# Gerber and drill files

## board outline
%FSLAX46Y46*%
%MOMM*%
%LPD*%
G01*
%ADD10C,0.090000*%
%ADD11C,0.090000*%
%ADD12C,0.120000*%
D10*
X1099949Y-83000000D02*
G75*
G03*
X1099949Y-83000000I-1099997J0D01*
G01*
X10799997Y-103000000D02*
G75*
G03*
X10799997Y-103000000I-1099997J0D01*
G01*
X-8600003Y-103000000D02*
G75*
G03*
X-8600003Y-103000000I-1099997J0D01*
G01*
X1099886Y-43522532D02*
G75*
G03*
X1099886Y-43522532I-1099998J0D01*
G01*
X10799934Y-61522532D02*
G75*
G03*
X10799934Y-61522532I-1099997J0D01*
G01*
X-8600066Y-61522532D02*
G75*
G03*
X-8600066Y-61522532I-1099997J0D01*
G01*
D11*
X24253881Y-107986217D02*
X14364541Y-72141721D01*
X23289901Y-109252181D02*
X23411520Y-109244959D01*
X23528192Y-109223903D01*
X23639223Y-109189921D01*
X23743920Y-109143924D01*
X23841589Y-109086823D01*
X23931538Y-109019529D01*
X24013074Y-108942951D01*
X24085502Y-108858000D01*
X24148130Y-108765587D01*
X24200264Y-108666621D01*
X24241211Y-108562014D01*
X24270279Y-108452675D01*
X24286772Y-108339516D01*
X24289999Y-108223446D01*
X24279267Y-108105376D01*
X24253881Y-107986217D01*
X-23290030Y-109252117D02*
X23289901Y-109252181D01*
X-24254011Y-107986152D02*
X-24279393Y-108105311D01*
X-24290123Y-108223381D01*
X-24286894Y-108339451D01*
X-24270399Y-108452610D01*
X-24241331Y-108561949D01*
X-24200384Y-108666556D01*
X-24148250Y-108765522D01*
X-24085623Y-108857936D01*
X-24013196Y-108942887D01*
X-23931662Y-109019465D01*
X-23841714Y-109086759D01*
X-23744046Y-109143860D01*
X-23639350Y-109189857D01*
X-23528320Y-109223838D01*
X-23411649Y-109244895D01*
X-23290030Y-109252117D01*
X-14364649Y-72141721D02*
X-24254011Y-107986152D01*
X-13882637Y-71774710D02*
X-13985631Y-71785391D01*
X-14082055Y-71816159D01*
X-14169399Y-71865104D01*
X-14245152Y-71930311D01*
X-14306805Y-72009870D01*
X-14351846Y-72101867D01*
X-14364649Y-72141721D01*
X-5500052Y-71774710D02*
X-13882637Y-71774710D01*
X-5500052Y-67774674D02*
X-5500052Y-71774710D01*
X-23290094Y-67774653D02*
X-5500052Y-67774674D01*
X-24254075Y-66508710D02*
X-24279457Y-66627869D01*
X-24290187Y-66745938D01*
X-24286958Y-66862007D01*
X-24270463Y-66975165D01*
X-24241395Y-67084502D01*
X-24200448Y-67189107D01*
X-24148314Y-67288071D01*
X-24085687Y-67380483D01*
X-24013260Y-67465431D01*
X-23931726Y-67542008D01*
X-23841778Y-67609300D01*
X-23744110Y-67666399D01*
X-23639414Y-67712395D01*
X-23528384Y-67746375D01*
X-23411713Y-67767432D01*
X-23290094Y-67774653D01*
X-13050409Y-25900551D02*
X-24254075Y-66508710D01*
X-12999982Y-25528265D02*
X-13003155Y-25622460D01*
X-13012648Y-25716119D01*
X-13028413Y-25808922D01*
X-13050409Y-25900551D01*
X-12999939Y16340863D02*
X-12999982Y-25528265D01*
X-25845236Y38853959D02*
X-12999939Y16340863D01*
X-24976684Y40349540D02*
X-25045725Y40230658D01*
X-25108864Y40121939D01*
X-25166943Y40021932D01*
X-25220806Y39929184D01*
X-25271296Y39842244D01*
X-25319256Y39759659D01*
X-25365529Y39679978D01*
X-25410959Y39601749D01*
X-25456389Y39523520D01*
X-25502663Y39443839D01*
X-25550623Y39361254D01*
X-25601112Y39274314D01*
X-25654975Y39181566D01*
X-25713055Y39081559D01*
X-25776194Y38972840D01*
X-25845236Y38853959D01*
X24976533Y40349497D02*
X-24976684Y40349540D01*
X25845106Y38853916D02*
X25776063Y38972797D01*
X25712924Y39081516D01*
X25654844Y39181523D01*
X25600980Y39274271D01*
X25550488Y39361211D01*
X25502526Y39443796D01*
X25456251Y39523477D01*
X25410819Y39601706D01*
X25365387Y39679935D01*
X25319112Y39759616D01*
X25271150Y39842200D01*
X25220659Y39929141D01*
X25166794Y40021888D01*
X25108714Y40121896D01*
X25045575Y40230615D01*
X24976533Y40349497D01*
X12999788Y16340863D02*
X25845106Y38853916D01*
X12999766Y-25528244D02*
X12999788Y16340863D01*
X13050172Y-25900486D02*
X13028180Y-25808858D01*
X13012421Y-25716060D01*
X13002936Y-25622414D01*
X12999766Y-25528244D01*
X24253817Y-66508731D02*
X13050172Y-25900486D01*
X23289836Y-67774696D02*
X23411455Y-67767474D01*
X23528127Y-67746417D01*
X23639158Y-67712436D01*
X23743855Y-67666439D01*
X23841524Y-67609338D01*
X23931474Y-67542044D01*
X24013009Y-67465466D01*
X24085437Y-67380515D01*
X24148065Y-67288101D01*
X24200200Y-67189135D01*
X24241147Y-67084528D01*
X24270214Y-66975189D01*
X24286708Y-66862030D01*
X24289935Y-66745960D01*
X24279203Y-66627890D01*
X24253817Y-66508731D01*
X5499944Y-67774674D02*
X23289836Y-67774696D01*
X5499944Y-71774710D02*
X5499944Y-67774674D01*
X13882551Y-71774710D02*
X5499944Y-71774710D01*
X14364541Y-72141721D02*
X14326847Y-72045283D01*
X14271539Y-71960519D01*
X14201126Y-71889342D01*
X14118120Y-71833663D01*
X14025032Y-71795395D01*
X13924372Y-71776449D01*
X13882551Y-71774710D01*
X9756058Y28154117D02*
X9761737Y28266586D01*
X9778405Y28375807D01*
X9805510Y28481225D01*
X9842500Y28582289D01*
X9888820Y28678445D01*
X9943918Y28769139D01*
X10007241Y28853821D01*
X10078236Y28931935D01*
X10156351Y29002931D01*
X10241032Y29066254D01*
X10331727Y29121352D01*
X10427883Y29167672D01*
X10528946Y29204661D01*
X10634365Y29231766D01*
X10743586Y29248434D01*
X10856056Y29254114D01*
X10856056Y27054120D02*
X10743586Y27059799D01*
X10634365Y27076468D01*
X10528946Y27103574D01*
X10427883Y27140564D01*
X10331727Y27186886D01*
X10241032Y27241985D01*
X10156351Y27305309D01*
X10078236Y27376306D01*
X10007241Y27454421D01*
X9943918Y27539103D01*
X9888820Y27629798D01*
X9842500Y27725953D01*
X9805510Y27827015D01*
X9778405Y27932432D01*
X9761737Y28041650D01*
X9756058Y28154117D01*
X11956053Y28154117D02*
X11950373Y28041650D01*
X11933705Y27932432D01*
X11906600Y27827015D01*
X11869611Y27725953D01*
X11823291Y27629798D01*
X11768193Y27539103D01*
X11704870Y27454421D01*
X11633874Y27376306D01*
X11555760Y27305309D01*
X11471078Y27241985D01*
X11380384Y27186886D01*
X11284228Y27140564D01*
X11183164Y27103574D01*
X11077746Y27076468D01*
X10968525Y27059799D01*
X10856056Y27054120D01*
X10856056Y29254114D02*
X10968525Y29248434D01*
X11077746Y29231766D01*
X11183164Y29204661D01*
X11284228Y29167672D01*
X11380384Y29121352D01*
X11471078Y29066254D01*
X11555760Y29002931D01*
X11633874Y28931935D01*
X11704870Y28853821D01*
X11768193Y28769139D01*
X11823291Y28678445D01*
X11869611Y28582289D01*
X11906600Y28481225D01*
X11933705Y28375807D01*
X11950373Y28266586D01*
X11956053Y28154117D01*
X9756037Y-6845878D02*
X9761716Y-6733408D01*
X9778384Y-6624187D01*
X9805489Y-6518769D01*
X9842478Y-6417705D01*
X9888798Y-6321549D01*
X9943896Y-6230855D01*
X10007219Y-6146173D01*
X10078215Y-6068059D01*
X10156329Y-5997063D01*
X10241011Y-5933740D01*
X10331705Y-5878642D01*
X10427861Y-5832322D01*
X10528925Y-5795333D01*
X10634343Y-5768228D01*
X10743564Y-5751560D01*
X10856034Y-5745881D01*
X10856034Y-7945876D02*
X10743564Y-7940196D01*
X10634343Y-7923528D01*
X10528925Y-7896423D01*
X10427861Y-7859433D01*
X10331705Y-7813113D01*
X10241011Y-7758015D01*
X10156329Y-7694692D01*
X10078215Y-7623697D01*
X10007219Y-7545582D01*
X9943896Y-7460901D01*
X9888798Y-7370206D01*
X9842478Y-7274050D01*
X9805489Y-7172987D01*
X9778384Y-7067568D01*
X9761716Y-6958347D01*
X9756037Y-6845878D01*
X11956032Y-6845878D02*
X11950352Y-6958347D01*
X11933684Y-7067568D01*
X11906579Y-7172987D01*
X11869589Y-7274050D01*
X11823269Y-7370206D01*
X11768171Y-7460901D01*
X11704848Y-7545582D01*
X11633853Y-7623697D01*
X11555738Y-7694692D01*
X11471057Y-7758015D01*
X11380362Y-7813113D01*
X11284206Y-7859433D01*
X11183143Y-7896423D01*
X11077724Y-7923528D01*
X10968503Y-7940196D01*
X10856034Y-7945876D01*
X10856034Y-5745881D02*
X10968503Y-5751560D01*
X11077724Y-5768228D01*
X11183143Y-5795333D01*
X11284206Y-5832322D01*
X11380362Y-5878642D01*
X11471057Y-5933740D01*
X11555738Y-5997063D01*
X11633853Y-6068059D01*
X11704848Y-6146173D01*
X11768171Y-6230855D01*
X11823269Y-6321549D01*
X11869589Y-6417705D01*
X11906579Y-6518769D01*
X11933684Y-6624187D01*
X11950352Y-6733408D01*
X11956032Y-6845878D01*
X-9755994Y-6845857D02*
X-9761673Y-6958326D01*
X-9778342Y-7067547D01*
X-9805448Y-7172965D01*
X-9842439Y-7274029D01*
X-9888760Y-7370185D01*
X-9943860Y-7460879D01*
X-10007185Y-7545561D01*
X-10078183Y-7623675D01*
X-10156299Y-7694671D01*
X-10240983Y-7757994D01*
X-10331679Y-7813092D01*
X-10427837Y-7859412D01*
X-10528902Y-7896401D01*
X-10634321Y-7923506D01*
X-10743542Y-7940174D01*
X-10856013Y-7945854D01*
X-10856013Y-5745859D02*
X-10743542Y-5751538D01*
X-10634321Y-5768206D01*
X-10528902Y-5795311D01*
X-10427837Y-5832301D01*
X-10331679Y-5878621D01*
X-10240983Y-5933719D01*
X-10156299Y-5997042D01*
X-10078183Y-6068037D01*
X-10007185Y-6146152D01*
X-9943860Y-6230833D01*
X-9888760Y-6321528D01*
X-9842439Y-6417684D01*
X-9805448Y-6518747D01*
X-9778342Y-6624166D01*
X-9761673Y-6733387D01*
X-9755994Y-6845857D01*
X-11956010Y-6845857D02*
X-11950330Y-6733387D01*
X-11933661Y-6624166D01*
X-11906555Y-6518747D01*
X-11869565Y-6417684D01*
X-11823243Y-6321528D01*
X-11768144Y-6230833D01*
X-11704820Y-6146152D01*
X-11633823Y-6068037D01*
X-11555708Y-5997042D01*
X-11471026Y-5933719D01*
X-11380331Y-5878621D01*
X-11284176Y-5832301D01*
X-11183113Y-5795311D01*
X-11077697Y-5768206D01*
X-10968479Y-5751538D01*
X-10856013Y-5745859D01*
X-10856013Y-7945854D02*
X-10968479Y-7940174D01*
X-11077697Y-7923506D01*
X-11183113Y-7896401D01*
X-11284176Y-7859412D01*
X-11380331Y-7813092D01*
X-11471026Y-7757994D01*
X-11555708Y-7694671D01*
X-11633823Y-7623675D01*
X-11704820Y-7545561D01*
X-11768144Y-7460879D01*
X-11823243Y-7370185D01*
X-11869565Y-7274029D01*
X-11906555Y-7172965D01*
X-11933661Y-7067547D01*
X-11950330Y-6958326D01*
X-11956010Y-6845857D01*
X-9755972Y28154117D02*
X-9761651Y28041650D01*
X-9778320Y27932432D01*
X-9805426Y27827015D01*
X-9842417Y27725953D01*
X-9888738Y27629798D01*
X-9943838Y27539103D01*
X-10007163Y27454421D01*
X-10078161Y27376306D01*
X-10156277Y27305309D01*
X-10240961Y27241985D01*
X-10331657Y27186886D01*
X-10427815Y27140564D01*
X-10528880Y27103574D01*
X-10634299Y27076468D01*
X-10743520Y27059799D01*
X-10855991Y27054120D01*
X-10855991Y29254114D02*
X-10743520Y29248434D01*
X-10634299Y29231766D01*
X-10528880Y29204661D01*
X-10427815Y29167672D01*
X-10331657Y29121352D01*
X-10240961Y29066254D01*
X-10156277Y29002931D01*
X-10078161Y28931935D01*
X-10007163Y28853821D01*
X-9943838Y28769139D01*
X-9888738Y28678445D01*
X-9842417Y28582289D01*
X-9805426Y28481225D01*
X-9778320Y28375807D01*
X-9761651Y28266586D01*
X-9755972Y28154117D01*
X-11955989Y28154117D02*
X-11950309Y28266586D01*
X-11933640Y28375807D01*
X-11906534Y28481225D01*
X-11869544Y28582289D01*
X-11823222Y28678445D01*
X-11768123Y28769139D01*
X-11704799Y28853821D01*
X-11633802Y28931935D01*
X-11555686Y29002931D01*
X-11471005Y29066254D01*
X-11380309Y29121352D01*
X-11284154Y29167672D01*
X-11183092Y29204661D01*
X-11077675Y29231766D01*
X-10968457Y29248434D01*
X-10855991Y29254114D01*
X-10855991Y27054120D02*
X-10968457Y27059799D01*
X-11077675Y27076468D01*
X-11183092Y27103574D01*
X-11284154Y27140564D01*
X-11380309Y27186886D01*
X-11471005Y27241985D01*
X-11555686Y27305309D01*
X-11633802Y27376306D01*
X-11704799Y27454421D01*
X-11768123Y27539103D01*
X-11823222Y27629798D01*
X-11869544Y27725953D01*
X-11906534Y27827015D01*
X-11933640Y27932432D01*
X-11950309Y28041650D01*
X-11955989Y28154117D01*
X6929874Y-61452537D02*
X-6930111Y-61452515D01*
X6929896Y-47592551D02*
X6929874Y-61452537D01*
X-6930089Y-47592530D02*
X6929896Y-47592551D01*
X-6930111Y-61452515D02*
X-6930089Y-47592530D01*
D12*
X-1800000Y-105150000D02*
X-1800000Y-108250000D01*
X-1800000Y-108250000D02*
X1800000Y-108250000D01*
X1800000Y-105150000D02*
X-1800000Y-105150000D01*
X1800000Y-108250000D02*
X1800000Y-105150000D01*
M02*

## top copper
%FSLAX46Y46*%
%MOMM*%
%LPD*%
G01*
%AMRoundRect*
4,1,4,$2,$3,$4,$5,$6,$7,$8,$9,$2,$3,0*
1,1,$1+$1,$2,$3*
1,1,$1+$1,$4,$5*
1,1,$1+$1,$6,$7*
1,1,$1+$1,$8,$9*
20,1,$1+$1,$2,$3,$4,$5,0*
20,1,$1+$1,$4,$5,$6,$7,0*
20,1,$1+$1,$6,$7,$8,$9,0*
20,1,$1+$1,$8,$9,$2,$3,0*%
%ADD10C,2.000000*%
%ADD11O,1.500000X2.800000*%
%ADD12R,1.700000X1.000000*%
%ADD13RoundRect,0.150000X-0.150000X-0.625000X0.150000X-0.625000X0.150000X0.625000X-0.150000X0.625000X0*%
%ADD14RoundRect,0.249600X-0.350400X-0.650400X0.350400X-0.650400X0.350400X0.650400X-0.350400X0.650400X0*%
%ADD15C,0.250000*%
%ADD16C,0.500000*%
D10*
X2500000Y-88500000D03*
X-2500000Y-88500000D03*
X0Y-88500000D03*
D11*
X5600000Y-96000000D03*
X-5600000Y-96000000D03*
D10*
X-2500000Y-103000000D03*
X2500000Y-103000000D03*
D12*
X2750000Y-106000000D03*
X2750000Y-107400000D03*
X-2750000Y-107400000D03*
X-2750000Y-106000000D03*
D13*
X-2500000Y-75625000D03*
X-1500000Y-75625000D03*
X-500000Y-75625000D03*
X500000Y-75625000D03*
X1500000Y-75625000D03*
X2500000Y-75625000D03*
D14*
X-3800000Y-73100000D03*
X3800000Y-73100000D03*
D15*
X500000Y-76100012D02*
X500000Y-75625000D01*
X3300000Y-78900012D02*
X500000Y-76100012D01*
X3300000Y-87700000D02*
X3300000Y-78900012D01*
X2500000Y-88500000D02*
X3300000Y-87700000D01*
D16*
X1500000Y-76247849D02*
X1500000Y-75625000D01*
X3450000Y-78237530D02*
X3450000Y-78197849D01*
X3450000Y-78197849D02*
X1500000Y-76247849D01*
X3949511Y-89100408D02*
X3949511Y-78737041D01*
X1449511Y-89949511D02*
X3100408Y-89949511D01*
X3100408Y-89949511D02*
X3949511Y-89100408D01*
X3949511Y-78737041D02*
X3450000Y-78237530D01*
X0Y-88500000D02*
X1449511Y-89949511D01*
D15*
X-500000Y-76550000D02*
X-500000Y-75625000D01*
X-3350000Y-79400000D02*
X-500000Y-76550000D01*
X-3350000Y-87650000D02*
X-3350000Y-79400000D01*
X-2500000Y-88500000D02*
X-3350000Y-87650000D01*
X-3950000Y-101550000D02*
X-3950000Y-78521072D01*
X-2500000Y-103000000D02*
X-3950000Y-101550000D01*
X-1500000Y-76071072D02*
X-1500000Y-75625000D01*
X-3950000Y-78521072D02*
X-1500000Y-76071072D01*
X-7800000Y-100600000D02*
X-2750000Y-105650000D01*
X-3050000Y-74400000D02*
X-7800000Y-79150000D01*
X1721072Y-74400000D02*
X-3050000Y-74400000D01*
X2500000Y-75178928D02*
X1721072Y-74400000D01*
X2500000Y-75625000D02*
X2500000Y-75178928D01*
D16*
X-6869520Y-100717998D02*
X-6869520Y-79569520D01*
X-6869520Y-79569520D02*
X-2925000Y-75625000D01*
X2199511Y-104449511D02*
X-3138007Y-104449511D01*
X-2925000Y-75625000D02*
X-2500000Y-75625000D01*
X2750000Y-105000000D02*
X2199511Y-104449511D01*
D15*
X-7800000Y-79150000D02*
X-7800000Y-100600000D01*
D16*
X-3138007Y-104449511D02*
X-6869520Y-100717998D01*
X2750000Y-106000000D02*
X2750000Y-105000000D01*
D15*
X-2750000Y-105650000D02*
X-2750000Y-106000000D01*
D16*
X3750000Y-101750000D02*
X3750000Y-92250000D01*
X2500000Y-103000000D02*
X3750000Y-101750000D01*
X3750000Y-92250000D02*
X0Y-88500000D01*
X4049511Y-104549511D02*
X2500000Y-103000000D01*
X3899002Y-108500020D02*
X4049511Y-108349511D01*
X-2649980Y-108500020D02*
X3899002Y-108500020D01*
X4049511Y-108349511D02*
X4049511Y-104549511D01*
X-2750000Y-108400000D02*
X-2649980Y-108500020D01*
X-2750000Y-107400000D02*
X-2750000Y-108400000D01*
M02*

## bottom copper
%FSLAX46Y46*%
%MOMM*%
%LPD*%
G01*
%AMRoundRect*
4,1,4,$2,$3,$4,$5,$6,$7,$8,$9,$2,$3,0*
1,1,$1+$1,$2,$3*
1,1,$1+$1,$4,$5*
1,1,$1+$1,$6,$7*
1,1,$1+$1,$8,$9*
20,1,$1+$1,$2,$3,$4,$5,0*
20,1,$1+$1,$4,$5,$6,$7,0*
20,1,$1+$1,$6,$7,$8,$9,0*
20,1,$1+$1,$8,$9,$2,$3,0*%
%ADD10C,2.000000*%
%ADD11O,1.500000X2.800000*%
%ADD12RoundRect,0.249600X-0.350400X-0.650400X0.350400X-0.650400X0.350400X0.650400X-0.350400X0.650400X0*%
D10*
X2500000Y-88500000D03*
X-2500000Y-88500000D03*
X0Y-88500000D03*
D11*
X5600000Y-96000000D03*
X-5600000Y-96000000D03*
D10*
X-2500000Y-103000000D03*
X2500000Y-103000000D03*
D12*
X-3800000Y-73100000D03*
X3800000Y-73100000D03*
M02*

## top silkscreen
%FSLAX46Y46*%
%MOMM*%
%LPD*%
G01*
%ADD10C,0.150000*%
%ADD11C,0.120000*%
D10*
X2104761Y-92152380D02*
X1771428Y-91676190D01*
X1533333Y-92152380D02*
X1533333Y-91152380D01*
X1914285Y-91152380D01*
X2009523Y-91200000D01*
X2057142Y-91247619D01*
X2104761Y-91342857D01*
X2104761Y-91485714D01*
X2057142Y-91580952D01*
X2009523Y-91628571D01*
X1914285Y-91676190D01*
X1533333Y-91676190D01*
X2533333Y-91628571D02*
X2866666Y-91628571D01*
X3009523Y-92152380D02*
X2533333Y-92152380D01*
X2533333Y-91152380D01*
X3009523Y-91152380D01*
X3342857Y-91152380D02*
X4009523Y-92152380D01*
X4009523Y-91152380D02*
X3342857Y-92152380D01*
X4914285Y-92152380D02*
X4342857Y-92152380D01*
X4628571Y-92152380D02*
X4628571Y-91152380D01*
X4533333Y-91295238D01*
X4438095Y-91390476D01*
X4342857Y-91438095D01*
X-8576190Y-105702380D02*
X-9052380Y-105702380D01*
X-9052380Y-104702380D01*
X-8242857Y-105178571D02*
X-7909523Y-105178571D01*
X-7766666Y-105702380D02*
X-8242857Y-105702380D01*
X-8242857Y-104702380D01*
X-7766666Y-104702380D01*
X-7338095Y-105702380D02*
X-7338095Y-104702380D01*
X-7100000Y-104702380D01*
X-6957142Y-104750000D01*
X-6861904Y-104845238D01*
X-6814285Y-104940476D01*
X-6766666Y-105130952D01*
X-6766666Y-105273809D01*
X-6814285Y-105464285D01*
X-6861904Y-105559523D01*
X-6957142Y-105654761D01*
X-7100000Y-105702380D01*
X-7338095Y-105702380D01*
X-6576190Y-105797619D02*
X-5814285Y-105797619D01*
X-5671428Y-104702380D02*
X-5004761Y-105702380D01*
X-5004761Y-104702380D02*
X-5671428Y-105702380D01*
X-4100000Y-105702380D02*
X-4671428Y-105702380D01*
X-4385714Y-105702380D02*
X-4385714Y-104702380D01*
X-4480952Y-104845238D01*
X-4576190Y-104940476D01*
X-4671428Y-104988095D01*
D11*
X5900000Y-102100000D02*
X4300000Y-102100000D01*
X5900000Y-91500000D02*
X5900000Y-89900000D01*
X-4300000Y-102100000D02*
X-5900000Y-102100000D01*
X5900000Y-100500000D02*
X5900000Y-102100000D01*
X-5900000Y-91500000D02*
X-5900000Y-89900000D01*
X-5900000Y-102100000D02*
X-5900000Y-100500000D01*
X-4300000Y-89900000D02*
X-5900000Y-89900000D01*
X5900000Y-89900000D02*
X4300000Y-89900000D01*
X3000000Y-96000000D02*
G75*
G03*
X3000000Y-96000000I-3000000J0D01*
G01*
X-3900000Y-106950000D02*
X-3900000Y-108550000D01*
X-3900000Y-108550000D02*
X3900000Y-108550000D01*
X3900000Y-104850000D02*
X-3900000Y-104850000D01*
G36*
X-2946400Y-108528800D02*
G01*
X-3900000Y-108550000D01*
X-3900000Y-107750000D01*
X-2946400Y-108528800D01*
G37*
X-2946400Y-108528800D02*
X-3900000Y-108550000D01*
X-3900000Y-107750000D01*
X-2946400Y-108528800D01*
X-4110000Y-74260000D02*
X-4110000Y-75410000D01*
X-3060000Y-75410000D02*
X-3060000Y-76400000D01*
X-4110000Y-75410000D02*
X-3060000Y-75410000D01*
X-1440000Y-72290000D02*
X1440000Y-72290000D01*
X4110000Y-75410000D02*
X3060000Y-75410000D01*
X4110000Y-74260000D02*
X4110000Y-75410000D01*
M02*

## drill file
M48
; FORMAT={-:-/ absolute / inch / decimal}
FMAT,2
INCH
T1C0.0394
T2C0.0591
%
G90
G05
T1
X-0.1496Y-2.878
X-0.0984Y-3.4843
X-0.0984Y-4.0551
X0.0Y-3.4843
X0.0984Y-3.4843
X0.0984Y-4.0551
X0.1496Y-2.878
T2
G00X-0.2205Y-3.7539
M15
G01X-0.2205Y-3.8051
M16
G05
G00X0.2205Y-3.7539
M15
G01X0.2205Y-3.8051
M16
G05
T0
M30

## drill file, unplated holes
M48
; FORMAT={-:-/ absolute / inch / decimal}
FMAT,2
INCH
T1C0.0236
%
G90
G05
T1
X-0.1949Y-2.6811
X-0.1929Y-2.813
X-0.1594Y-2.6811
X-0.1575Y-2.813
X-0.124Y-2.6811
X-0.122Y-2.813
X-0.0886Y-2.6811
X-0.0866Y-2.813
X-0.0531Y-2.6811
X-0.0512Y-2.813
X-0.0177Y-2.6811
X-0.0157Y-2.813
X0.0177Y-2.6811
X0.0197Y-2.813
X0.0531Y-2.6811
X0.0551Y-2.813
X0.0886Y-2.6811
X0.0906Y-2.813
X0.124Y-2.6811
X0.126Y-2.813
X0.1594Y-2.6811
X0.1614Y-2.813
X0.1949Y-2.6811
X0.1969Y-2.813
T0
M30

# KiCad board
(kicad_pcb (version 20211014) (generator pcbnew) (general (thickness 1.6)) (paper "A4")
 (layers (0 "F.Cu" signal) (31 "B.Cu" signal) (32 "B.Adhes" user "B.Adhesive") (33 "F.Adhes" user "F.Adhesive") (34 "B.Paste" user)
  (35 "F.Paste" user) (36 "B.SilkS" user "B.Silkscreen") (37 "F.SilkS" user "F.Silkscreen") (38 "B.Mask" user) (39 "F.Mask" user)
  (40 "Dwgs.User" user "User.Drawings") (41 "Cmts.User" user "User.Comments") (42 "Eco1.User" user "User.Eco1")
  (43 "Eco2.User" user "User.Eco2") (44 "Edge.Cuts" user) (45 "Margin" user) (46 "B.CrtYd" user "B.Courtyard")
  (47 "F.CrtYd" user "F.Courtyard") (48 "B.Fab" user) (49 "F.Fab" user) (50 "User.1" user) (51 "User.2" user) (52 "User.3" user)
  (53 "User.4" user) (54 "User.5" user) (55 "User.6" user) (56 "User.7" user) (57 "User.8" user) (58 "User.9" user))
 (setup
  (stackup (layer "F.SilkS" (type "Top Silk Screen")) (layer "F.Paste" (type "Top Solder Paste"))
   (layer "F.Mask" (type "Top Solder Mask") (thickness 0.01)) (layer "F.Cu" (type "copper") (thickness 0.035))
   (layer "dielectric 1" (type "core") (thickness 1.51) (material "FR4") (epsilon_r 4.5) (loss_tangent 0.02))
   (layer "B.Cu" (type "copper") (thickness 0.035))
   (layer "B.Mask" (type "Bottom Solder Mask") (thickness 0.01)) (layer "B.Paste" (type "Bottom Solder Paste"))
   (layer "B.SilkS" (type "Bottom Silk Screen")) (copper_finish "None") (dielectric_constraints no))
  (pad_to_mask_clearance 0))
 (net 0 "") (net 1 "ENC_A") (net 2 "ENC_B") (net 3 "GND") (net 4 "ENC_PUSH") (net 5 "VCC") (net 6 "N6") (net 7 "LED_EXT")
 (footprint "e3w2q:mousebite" (layer "F.Cu") (at -5.2 71.75)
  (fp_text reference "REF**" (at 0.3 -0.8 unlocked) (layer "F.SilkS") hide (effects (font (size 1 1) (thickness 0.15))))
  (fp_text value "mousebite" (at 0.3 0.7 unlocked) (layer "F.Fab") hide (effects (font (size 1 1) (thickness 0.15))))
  (pad "" np_thru_hole circle (at 3 -0.3) (size 0.6 0.6) (drill 0.6) (layers F&B.Cu *.Mask))
  (pad "" np_thru_hole circle (at 7.5 -0.3) (size 0.6 0.6) (drill 0.6) (layers F&B.Cu *.Mask))
  (pad "" np_thru_hole circle (at 10.2 -0.3) (size 0.6 0.6) (drill 0.6) (layers F&B.Cu *.Mask))
  (pad "" np_thru_hole circle (at 1.2 -0.3) (size 0.6 0.6) (drill 0.6) (layers F&B.Cu *.Mask))
  (pad "" np_thru_hole circle (at 4.8 -0.3) (size 0.6 0.6) (drill 0.6) (layers F&B.Cu *.Mask))
  (pad "" np_thru_hole circle (at 0.3 -0.3) (size 0.6 0.6) (drill 0.6) (layers F&B.Cu *.Mask))
  (pad "" np_thru_hole circle (at 2.1 -0.3) (size 0.6 0.6) (drill 0.6) (layers F&B.Cu *.Mask))
  (pad "" np_thru_hole circle (at 5.7 -0.3) (size 0.6 0.6) (drill 0.6) (layers F&B.Cu *.Mask))
  (pad "" np_thru_hole circle (at 6.6 -0.3) (size 0.6 0.6) (drill 0.6) (layers F&B.Cu *.Mask))
  (pad "" np_thru_hole circle (at 3.9 -0.3) (size 0.6 0.6) (drill 0.6) (layers F&B.Cu *.Mask))
  (pad "" np_thru_hole circle (at 9.3 -0.3) (size 0.6 0.6) (drill 0.6) (layers F&B.Cu *.Mask))
  (pad "" np_thru_hole circle (at 8.4 -0.3) (size 0.6 0.6) (drill 0.6) (layers F&B.Cu *.Mask)))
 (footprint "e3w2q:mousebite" (layer "F.Cu") (at -5.25 68.4)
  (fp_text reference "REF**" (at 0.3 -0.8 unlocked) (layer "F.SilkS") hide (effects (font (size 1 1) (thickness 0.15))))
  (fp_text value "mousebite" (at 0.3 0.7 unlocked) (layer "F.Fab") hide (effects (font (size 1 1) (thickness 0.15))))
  (pad "" np_thru_hole circle (at 4.8 -0.3) (size 0.6 0.6) (drill 0.6) (layers F&B.Cu *.Mask))
  (pad "" np_thru_hole circle (at 3.9 -0.3) (size 0.6 0.6) (drill 0.6) (layers F&B.Cu *.Mask))
  (pad "" np_thru_hole circle (at 6.6 -0.3) (size 0.6 0.6) (drill 0.6) (layers F&B.Cu *.Mask))
  (pad "" np_thru_hole circle (at 1.2 -0.3) (size 0.6 0.6) (drill 0.6) (layers F&B.Cu *.Mask))
  (pad "" np_thru_hole circle (at 5.7 -0.3) (size 0.6 0.6) (drill 0.6) (layers F&B.Cu *.Mask))
  (pad "" np_thru_hole circle (at 8.4 -0.3) (size 0.6 0.6) (drill 0.6) (layers F&B.Cu *.Mask))
  (pad "" np_thru_hole circle (at 10.2 -0.3) (size 0.6 0.6) (drill 0.6) (layers F&B.Cu *.Mask))
  (pad "" np_thru_hole circle (at 0.3 -0.3) (size 0.6 0.6) (drill 0.6) (layers F&B.Cu *.Mask))
  (pad "" np_thru_hole circle (at 2.1 -0.3) (size 0.6 0.6) (drill 0.6) (layers F&B.Cu *.Mask))
  (pad "" np_thru_hole circle (at 7.5 -0.3) (size 0.6 0.6) (drill 0.6) (layers F&B.Cu *.Mask))
  (pad "" np_thru_hole circle (at 9.3 -0.3) (size 0.6 0.6) (drill 0.6) (layers F&B.Cu *.Mask))
  (pad "" np_thru_hole circle (at 3 -0.3) (size 0.6 0.6) (drill 0.6) (layers F&B.Cu *.Mask)))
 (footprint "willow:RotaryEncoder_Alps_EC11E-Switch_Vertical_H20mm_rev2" (layer "F.Cu") (at 0 96 -90)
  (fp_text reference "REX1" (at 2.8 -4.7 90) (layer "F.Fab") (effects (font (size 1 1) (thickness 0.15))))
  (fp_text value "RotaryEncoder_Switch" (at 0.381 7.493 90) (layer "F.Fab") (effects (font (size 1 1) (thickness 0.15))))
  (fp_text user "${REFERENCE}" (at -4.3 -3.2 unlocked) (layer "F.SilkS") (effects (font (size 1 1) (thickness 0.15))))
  (fp_line (start -4.5 5.9) (end -6.1 5.9) (layer "F.SilkS") (width 0.12))
  (fp_line (start 6.1 4.3) (end 6.1 5.9) (layer "F.SilkS") (width 0.12))
  (fp_line (start 6.1 -5.9) (end 6.1 -4.3) (layer "F.SilkS") (width 0.12))
  (fp_line (start -6.1 -5.9) (end -6.1 -4.3) (layer "F.SilkS") (width 0.12))
  (fp_line (start -6.1 4.3) (end -6.1 5.9) (layer "F.SilkS") (width 0.12))
  (fp_line (start -4.5 -5.9) (end -6.1 -5.9) (layer "F.SilkS") (width 0.12))
  (fp_line (start 4.5 -5.9) (end 6.1 -5.9) (layer "F.SilkS") (width 0.12))
  (fp_line (start 6.1 5.9) (end 4.5 5.9) (layer "F.SilkS") (width 0.12))
  (fp_circle (center 0 0) (end 3 0) (layer "F.SilkS") (width 0.12) (fill none))
  (pad "A" thru_hole circle (at -7.5 -2.5 270) (size 2 2) (drill 1) (layers *.Cu *.Mask) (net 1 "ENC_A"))
  (pad "B" thru_hole circle (at -7.5 2.5 270) (size 2 2) (drill 1) (layers *.Cu *.Mask) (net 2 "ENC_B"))
  (pad "C" thru_hole circle (at -7.5 0 270) (size 2 2) (drill 1) (layers *.Cu *.Mask) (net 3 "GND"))
  (pad "MP" thru_hole oval (at 0 -5.6 270) (size 2.8 1.5) (drill oval 2.8 1.5) (layers *.Cu *.Mask))
  (pad "MP" thru_hole oval (at 0 5.6 270) (size 2.8 1.5) (drill oval 2.8 1.5) (layers *.Cu *.Mask))
  (pad "S1" thru_hole circle (at 7 2.5 270) (size 2 2) (drill 1) (layers *.Cu *.Mask) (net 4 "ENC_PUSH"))
  (pad "S2" thru_hole circle (at 7 -2.5 270) (size 2 2) (drill 1) (layers *.Cu *.Mask) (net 3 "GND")))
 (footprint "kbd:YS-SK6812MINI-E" (layer "F.Cu") (at 0 106.7)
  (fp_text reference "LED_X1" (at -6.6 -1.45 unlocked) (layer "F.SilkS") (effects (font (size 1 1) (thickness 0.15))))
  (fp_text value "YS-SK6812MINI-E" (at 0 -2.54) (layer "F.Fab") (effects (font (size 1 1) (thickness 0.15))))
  (fp_line (start -3.9 0.25) (end -3.9 1.85) (layer "F.SilkS") (width 0.12))
  (fp_line (start 3.9 -1.85) (end -3.9 -1.85) (layer "F.SilkS") (width 0.12))
  (fp_line (start -3.9 1.85) (end 3.9 1.85) (layer "F.SilkS") (width 0.12))
  (fp_poly (pts (xy -2.9464 1.8288) (xy -3.9 1.85) (xy -3.9 1.05)) (layer "F.SilkS") (width 0.12) (fill solid))
  (fp_line (start 1.8 -1.55) (end -1.8 -1.55) (layer "Edge.Cuts") (width 0.12))
  (fp_line (start -1.8 1.55) (end 1.8 1.55) (layer "Edge.Cuts") (width 0.12))
  (fp_line (start -1.8 -1.55) (end -1.8 1.55) (layer "Edge.Cuts") (width 0.12))
  (fp_line (start 1.8 1.55) (end 1.8 -1.55) (layer "Edge.Cuts") (width 0.12))
  (pad "1" smd rect (at 2.75 -0.7) (size 1.7 1) (layers "F.Cu" "F.Paste" "F.Mask") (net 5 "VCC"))
  (pad "2" smd rect (at 2.75 0.7) (size 1.7 1) (layers "F.Cu" "F.Paste" "F.Mask") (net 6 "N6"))
  (pad "3" smd rect (at -2.75 0.7) (size 1.7 1) (layers "F.Cu" "F.Paste" "F.Mask") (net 3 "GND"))
  (pad "4" smd rect (at -2.75 -0.7) (size 1.7 1) (layers "F.Cu" "F.Paste" "F.Mask") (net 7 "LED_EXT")))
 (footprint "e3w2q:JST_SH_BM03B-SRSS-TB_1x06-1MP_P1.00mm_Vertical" (layer "F.Cu") (at 0 74.3)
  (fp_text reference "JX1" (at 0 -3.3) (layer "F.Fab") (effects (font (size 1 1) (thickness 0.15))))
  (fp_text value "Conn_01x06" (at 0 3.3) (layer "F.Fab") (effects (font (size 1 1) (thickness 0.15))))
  (fp_line (start -4.11 -0.04) (end -4.11 1.11) (layer "F.SilkS") (width 0.12))
  (fp_line (start 4.11 1.11) (end 3.06 1.11) (layer "F.SilkS") (width 0.12))
  (fp_line (start -3.06 1.11) (end -3.06 2.1) (layer "F.SilkS") (width 0.12))
  (fp_line (start 4.11 -0.04) (end 4.11 1.11) (layer "F.SilkS") (width 0.12))
  (fp_line (start -1.44 -2.01) (end 1.44 -2.01) (layer "F.SilkS") (width 0.12))
  (fp_line (start -4.11 1.11) (end -3.06 1.11) (layer "F.SilkS") (width 0.12))
  (pad "1" smd roundrect (at -2.5 1.325) (size 0.6 1.55) (layers "F.Cu" "F.Paste" "F.Mask") (roundrect_rratio 0.25) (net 5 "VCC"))
  (pad "2" smd roundrect (at -1.5 1.325) (size 0.6 1.55) (layers "F.Cu" "F.Paste" "F.Mask") (roundrect_rratio 0.25) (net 4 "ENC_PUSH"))
  (pad "3" smd roundrect (at -0.5 1.325) (size 0.6 1.55) (layers "F.Cu" "F.Paste" "F.Mask") (roundrect_rratio 0.25) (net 2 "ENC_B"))
  (pad "4" smd roundrect (at 0.5 1.325) (size 0.6 1.55) (layers "F.Cu" "F.Paste" "F.Mask") (roundrect_rratio 0.25) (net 1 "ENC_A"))
  (pad "5" smd roundrect (at 1.5 1.325) (size 0.6 1.55) (layers "F.Cu" "F.Paste" "F.Mask") (roundrect_rratio 0.25) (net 3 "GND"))
  (pad "6" smd roundrect (at 2.5 1.325) (size 0.6 1.55) (layers "F.Cu" "F.Paste" "F.Mask") (roundrect_rratio 0.25) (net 7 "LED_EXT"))
  (pad "MP" thru_hole roundrect (at -3.8 -1.2) (size 1.2 1.8) (drill 1) (layers *.Cu *.Mask) (roundrect_rratio 0.208))
  (pad "MP" thru_hole roundrect (at 3.8 -1.2) (size 1.2 1.8) (drill 1) (layers *.Cu *.Mask) (roundrect_rratio 0.208)))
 (gr_circle (center 9.7 103) (end 10.799997 103) (layer "Edge.Cuts") (width 0.09) (fill none))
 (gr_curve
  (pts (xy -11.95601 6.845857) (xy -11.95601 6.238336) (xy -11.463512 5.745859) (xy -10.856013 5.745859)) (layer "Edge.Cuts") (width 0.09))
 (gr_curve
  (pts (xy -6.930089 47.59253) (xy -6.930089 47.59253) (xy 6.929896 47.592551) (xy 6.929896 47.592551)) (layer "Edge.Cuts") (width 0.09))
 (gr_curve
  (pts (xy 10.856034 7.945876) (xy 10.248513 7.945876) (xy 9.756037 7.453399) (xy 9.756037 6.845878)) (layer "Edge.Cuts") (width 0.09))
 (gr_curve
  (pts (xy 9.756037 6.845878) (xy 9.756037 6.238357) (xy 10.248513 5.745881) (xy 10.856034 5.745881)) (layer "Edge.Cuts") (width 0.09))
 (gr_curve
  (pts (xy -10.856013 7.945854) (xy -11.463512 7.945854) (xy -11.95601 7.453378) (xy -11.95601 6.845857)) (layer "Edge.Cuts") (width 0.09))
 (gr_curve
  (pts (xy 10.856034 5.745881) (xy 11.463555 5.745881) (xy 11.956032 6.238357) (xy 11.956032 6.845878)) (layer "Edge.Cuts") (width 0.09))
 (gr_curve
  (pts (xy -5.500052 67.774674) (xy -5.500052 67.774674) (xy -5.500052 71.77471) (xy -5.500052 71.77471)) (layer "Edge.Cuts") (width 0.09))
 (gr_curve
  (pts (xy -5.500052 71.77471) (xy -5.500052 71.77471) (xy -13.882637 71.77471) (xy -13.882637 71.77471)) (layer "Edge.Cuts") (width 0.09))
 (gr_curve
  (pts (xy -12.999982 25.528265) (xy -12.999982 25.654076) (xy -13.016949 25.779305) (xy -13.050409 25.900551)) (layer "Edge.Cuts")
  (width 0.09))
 (gr_circle (center -9.7 103) (end -8.600003 103) (layer "Edge.Cuts") (width 0.09) (fill none))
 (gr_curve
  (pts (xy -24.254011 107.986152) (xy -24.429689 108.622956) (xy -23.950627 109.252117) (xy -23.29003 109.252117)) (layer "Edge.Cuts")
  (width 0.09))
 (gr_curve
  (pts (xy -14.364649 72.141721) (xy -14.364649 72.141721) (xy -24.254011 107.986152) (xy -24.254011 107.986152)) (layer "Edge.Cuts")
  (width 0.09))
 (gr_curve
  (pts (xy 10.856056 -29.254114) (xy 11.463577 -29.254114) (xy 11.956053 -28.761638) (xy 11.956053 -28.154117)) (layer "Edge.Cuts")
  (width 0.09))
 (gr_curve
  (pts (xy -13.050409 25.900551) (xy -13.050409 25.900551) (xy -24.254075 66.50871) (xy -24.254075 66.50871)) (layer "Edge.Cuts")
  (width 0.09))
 (gr_circle (center -0.000112 43.522532) (end 1.099886 43.522532) (layer "Edge.Cuts") (width 0.09) (fill none))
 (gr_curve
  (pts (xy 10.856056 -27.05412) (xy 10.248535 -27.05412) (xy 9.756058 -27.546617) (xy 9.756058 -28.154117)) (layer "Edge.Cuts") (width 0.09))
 (gr_circle (center -9.700063 61.522532) (end -8.600066 61.522532) (layer "Edge.Cuts") (width 0.09) (fill none))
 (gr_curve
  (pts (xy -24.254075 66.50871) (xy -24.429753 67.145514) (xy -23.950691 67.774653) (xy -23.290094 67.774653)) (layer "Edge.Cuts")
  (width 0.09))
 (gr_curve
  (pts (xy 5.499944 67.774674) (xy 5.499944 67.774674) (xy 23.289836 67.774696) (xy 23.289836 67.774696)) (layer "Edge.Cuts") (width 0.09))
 (gr_circle (center -0.000048 83) (end 1.099949 83) (layer "Edge.Cuts") (width 0.09) (fill none))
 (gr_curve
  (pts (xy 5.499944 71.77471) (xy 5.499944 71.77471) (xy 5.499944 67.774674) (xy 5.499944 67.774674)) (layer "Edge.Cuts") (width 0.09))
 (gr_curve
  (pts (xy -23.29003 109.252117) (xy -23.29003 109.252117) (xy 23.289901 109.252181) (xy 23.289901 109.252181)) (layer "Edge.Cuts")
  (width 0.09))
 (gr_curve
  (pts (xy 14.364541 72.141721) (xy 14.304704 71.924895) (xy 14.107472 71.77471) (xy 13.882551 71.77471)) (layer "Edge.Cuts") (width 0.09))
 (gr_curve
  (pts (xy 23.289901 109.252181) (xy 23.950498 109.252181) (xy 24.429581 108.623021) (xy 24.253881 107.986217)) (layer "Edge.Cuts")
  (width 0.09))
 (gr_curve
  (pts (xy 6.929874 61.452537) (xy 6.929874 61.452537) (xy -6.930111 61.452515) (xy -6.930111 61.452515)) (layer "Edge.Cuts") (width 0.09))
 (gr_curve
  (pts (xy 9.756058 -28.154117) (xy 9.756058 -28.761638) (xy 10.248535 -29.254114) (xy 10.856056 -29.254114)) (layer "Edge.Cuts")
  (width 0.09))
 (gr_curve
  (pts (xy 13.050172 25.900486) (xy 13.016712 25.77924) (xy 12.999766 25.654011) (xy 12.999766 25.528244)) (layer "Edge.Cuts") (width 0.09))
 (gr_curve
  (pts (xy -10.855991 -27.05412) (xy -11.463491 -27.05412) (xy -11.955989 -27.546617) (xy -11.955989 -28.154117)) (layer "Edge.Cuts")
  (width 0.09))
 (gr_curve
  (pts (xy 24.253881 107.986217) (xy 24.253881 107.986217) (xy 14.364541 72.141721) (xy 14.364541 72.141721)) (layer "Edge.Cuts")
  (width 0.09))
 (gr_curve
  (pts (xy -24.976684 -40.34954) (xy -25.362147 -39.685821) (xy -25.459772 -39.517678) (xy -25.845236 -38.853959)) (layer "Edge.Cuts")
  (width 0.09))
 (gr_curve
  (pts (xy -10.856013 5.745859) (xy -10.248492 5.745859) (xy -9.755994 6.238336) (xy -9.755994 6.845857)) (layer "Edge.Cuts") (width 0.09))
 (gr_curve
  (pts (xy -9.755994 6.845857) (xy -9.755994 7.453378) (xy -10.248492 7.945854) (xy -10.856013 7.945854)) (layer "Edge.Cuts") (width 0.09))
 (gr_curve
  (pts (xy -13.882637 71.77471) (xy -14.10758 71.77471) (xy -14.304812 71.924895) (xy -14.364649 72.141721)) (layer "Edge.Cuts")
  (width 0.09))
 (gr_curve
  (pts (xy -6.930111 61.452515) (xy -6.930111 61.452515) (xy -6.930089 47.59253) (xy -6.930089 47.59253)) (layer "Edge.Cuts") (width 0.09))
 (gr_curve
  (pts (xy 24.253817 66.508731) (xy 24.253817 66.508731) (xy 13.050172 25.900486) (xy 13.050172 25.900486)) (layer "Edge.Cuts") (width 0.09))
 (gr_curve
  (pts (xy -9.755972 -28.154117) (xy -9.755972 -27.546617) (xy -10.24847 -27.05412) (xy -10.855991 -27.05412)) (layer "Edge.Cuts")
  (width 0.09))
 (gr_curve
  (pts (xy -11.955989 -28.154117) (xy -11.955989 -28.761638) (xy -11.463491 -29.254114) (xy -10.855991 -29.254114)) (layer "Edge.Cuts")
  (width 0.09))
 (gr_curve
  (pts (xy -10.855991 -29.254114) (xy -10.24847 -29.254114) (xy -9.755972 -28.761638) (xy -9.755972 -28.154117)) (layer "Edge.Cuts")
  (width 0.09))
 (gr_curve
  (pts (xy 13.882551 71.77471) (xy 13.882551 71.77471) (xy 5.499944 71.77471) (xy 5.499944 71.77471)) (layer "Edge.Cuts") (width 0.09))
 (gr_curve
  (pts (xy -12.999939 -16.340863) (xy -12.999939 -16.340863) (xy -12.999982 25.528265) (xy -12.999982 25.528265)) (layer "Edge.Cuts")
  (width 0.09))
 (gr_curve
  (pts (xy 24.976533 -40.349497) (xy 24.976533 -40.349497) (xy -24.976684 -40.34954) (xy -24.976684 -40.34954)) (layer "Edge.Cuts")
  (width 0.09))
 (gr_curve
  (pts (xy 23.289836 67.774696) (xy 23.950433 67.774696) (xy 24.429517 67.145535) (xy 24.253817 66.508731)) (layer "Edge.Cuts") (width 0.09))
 (gr_circle (center 9.699937 61.522532) (end 10.799934 61.522532) (layer "Edge.Cuts") (width 0.09) (fill none))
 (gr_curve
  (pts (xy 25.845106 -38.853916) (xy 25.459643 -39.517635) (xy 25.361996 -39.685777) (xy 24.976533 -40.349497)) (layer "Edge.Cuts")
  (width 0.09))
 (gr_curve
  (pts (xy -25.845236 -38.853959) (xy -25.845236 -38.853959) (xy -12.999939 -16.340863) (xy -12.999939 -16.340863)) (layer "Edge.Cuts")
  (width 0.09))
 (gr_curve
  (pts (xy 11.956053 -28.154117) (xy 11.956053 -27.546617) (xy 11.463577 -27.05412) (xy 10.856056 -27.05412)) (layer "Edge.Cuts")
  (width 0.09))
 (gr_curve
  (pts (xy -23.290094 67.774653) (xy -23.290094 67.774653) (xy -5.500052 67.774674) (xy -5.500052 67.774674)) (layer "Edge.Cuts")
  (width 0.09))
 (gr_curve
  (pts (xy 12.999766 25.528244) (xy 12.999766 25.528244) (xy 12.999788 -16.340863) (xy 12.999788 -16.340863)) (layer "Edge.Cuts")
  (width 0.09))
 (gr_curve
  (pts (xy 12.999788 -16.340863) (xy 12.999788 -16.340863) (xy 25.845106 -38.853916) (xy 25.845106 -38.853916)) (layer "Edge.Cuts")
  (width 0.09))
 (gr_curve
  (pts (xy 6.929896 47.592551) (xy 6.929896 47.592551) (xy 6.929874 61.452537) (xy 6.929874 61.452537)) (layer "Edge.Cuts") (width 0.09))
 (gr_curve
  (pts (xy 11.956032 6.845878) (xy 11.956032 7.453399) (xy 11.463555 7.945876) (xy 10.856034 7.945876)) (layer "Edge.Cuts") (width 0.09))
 (segment (start -6.86952 79.56952) (end -2.925 75.625) (width 0.5) (layer "F.Cu") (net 5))
 (segment (start 2.75 105) (end 2.199511 104.449511) (width 0.5) (layer "F.Cu") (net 5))
 (segment (start -6.86952 100.717998) (end -6.86952 79.56952) (width 0.5) (layer "F.Cu") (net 5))
 (segment (start -2.925 75.625) (end -2.5 75.625) (width 0.5) (layer "F.Cu") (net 5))
 (segment (start -3.138007 104.449511) (end -6.86952 100.717998) (width 0.5) (layer "F.Cu") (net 5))
 (segment (start 2.75 106) (end 2.75 105) (width 0.5) (layer "F.Cu") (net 5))
 (segment (start 2.199511 104.449511) (end -3.138007 104.449511) (width 0.5) (layer "F.Cu") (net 5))
 (segment (start -3.95 101.55) (end -3.95 78.521072) (width 0.25) (layer "F.Cu") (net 4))
 (segment (start -3.95 78.521072) (end -1.5 76.071072) (width 0.25) (layer "F.Cu") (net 4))
 (segment (start -1.5 76.071072) (end -1.5 75.625) (width 0.25) (layer "F.Cu") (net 4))
 (segment (start -2.5 103) (end -3.95 101.55) (width 0.25) (layer "F.Cu") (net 4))
 (segment (start -3.35 79.4) (end -0.5 76.55) (width 0.25) (layer "F.Cu") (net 2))
 (segment (start -2.5 88.5) (end -3.35 87.65) (width 0.25) (layer "F.Cu") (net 2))
 (segment (start -3.35 87.65) (end -3.35 79.4) (width 0.25) (layer "F.Cu") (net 2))
 (segment (start -0.5 76.55) (end -0.5 75.625) (width 0.25) (layer "F.Cu") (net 2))
 (segment (start 3.3 87.7) (end 3.3 78.900012) (width 0.25) (layer "F.Cu") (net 1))
 (segment (start 0.5 76.100012) (end 0.5 75.625) (width 0.25) (layer "F.Cu") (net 1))
 (segment (start 3.3 78.900012) (end 0.5 76.100012) (width 0.25) (layer "F.Cu") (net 1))
 (segment (start 2.5 88.5) (end 3.3 87.7) (width 0.25) (layer "F.Cu") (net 1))
 (segment (start -2.64998 108.50002) (end 3.899002 108.50002) (width 0.5) (layer "F.Cu") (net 3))
 (segment (start 3.75 101.75) (end 3.75 92.25) (width 0.5) (layer "F.Cu") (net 3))
 (segment (start 1.449511 89.949511) (end 3.100408 89.949511) (width 0.5) (layer "F.Cu") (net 3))
 (segment (start 1.5 76.247849) (end 1.5 75.625) (width 0.5) (layer "F.Cu") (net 3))
 (segment (start 3.45 78.197849) (end 1.5 76.247849) (width 0.5) (layer "F.Cu") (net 3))
 (segment (start 2.5 103) (end 3.75 101.75) (width 0.5) (layer "F.Cu") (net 3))
 (segment (start 4.049511 108.349511) (end 4.049511 104.549511) (width 0.5) (layer "F.Cu") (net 3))
 (segment (start -2.75 107.4) (end -2.75 108.4) (width 0.5) (layer "F.Cu") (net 3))
 (segment (start 3.75 92.25) (end 0 88.5) (width 0.5) (layer "F.Cu") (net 3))
 (segment (start 3.949511 89.100408) (end 3.949511 78.737041) (width 0.5) (layer "F.Cu") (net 3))
 (segment (start -2.75 108.4) (end -2.64998 108.50002) (width 0.5) (layer "F.Cu") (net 3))
 (segment (start 3.45 78.23753) (end 3.45 78.197849) (width 0.5) (layer "F.Cu") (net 3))
 (segment (start 3.100408 89.949511) (end 3.949511 89.100408) (width 0.5) (layer "F.Cu") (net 3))
 (segment (start 3.899002 108.50002) (end 4.049511 108.349511) (width 0.5) (layer "F.Cu") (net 3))
 (segment (start 3.949511 78.737041) (end 3.45 78.23753) (width 0.5) (layer "F.Cu") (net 3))
 (segment (start 4.049511 104.549511) (end 2.5 103) (width 0.5) (layer "F.Cu") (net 3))
 (segment (start 0 88.5) (end 1.449511 89.949511) (width 0.5) (layer "F.Cu") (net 3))
 (segment (start -7.8 79.15) (end -7.8 100.6) (width 0.25) (layer "F.Cu") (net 7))
 (segment (start -3.05 74.4) (end -7.8 79.15) (width 0.25) (layer "F.Cu") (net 7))
 (segment (start 2.5 75.625) (end 2.5 75.178928) (width 0.25) (layer "F.Cu") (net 7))
 (segment (start 2.5 75.178928) (end 1.721072 74.4) (width 0.25) (layer "F.Cu") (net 7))
 (segment (start 1.721072 74.4) (end -3.05 74.4) (width 0.25) (layer "F.Cu") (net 7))
 (segment (start -7.8 100.6) (end -2.75 105.65) (width 0.25) (layer "F.Cu") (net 7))
 (segment (start -2.75 105.65) (end -2.75 106) (width 0.25) (layer "F.Cu") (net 7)))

